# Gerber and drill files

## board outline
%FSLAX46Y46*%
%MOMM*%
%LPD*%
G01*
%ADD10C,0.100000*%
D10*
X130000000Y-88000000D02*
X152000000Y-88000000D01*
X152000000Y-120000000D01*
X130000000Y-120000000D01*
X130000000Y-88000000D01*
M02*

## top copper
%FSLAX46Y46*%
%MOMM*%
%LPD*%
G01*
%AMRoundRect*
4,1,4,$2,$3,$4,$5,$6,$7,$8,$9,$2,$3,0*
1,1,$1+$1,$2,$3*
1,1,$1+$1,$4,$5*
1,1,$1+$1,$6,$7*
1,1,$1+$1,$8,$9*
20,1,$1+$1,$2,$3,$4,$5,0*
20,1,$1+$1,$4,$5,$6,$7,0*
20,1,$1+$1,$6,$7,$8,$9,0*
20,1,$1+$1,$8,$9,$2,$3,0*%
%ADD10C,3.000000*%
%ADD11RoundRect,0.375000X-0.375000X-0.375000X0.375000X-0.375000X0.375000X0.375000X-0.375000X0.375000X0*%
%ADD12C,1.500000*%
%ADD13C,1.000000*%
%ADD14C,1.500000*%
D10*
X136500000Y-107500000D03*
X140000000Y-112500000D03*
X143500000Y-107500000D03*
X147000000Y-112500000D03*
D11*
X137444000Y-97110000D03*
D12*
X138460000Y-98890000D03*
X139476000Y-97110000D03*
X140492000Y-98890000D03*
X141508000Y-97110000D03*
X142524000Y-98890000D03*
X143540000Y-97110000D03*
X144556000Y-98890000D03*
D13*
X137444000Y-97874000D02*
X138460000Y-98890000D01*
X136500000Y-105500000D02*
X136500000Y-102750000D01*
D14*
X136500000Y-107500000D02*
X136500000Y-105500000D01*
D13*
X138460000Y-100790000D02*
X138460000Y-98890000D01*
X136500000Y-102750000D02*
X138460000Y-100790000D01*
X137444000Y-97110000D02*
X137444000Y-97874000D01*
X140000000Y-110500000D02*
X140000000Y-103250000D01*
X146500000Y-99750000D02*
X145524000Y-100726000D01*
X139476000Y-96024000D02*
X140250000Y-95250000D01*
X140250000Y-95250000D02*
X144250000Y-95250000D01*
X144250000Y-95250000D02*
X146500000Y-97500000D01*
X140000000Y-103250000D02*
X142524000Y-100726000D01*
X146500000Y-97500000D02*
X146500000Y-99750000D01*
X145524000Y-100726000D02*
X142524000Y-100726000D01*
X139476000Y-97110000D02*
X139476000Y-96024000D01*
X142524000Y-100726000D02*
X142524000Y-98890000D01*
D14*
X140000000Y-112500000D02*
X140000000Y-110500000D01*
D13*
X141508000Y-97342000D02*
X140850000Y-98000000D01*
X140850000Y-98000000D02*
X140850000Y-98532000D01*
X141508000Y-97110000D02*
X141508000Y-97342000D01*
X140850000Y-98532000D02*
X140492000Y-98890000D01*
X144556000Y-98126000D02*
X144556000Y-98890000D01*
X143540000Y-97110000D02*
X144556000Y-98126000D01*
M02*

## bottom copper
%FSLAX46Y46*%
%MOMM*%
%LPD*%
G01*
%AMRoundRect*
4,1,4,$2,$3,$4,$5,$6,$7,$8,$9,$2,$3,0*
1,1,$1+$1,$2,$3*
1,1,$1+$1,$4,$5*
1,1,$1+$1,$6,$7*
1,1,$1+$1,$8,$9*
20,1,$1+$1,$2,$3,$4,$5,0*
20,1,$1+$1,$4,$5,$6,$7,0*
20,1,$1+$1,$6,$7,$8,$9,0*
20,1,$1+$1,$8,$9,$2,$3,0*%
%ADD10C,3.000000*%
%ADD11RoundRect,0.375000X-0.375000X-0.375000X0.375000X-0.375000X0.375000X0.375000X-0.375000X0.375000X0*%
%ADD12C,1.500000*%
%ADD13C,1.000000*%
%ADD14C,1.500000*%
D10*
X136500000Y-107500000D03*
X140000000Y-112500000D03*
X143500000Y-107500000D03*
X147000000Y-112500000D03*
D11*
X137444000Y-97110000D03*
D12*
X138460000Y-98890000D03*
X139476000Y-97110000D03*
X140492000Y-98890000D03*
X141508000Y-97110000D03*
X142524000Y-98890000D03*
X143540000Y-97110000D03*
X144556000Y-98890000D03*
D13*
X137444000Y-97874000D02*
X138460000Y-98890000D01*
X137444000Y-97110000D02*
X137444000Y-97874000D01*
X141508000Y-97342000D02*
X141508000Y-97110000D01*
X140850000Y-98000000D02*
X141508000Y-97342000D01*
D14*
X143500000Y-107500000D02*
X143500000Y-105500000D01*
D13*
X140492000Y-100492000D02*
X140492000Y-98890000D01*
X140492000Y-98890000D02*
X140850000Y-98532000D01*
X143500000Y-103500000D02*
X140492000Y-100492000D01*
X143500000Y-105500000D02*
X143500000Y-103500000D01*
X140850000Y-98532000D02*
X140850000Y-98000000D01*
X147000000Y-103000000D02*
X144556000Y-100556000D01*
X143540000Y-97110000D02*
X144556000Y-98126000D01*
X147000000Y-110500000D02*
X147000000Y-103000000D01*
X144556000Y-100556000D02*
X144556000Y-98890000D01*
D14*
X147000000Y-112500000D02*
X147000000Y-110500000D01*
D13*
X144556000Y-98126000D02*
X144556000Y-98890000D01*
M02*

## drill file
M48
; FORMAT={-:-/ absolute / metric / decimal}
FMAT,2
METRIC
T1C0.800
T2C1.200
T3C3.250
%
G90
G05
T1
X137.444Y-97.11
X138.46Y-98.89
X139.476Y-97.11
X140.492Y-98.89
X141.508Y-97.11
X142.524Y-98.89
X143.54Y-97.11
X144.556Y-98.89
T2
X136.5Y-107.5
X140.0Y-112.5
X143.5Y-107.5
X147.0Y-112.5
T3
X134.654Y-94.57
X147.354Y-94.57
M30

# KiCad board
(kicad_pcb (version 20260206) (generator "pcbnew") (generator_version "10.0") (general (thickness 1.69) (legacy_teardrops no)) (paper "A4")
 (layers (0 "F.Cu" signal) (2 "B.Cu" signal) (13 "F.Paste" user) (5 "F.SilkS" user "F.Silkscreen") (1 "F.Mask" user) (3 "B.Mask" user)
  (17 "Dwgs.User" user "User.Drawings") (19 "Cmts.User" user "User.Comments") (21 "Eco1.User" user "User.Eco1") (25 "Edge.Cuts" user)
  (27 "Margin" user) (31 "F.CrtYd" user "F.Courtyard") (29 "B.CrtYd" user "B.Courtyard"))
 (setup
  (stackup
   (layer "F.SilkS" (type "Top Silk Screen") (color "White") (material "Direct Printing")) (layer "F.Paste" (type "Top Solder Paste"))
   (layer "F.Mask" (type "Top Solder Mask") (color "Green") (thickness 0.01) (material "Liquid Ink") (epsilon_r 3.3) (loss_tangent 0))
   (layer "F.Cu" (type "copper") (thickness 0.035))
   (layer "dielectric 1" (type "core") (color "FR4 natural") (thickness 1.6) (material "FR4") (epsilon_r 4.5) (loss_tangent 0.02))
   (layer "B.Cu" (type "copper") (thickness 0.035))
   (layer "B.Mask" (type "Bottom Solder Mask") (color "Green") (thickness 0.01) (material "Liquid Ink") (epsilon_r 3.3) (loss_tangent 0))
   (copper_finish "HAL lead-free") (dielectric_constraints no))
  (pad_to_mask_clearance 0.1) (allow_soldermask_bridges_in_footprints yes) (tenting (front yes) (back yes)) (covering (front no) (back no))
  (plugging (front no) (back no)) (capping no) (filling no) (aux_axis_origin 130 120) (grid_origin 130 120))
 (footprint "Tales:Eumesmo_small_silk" (layer "F.Cu") (at 148.5 101 90)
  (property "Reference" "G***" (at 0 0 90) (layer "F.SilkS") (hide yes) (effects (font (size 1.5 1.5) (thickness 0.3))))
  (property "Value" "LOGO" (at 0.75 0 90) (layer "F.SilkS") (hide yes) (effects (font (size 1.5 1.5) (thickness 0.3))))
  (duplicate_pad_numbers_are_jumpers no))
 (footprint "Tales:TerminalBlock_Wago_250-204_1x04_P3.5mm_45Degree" (layer "F.Cu") (at 141.75 110)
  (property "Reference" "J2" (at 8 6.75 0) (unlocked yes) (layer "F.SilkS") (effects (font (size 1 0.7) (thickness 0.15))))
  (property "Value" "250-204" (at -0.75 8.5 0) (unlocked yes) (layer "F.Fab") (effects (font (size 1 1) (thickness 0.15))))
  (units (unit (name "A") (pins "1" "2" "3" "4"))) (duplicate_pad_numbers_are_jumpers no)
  (pad "1" thru_hole circle (at -5.25 -2.5) (size 3 3) (drill 1.2) (layers "*.Cu" "*.Mask") (remove_unused_layers no) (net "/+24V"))
  (pad "2" thru_hole circle (at -1.75 2.5) (size 3 3) (drill 1.2) (layers "*.Cu" "*.Mask") (remove_unused_layers no) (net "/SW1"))
  (pad "3" thru_hole circle (at 1.75 -2.5) (size 3 3) (drill 1.2) (layers "*.Cu" "*.Mask") (remove_unused_layers no) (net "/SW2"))
  (pad "4" thru_hole circle (at 5.25 2.5) (size 3 3) (drill 1.2) (layers "*.Cu" "*.Mask") (remove_unused_layers no) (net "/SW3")))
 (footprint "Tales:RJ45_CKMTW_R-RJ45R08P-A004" (layer "F.Cu") (at 141 98 180)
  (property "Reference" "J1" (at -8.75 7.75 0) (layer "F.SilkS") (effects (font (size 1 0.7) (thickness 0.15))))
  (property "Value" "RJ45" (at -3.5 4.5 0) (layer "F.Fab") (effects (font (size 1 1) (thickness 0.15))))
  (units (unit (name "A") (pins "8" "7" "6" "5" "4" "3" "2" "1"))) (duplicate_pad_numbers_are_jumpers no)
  (pad "" np_thru_hole circle (at -6.354 3.43) (size 3.25 3.25) (drill 3.25) (layers "*.Cu" "*.Mask"))
  (pad "" np_thru_hole circle (at 6.346 3.43) (size 3.25 3.25) (drill 3.25) (layers "*.Cu" "*.Mask"))
  (pad "1" thru_hole roundrect (at 3.556 0.89) (size 1.5 1.5) (drill 0.8) (layers "*.Cu" "*.Mask") (remove_unused_layers no)
   (roundrect_rratio 0.25) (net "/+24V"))
  (pad "2" thru_hole circle (at 2.54 -0.89) (size 1.5 1.5) (drill 0.8) (layers "*.Cu" "*.Mask") (remove_unused_layers no) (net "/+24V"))
  (pad "3" thru_hole circle (at 1.524 0.89) (size 1.5 1.5) (drill 0.8) (layers "*.Cu" "*.Mask") (remove_unused_layers no) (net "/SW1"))
  (pad "4" thru_hole circle (at 0.508 -0.89) (size 1.5 1.5) (drill 0.8) (layers "*.Cu" "*.Mask") (remove_unused_layers no) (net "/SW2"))
  (pad "5" thru_hole circle (at -0.508 0.89) (size 1.5 1.5) (drill 0.8) (layers "*.Cu" "*.Mask") (remove_unused_layers no) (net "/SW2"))
  (pad "6" thru_hole circle (at -1.524 -0.89) (size 1.5 1.5) (drill 0.8) (layers "*.Cu" "*.Mask") (remove_unused_layers no) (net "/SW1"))
  (pad "7" thru_hole circle (at -2.54 0.89) (size 1.5 1.5) (drill 0.8) (layers "*.Cu" "*.Mask") (remove_unused_layers no) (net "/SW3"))
  (pad "8" thru_hole circle (at -3.556 -0.89) (size 1.5 1.5) (drill 0.8) (layers "*.Cu" "*.Mask") (remove_unused_layers no) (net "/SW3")))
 (gr_rect (start 130 88) (end 152 120) (stroke (width 0.1) (type default)) (fill no) (layer "Edge.Cuts"))
 (segment (start 137.444 97.874) (end 138.46 98.89) (width 1) (layer "F.Cu") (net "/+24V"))
 (segment (start 136.5 105.5) (end 136.5 102.75) (width 1) (layer "F.Cu") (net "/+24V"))
 (segment (start 136.5 107.5) (end 136.5 105.5) (width 1.5) (layer "F.Cu") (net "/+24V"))
 (segment (start 138.46 100.79) (end 138.46 98.89) (width 1) (layer "F.Cu") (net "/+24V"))
 (segment (start 136.5 102.75) (end 138.46 100.79) (width 1) (layer "F.Cu") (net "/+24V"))
 (segment (start 137.444 97.11) (end 137.444 97.874) (width 1) (layer "F.Cu") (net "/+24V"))
 (segment (start 137.444 97.874) (end 138.46 98.89) (width 1) (layer "B.Cu") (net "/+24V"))
 (segment (start 137.444 97.11) (end 137.444 97.874) (width 1) (layer "B.Cu") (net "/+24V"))
 (segment (start 140 110.5) (end 140 103.25) (width 1) (layer "F.Cu") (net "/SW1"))
 (segment (start 146.5 99.75) (end 145.524 100.726) (width 1) (layer "F.Cu") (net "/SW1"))
 (segment (start 139.476 96.024) (end 140.25 95.25) (width 1) (layer "F.Cu") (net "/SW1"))
 (segment (start 140.25 95.25) (end 144.25 95.25) (width 1) (layer "F.Cu") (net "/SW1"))
 (segment (start 144.25 95.25) (end 146.5 97.5) (width 1) (layer "F.Cu") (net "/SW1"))
 (segment (start 140 103.25) (end 142.524 100.726) (width 1) (layer "F.Cu") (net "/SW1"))
 (segment (start 146.5 97.5) (end 146.5 99.75) (width 1) (layer "F.Cu") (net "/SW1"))
 (segment (start 145.524 100.726) (end 142.524 100.726) (width 1) (layer "F.Cu") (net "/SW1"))
 (segment (start 139.476 97.11) (end 139.476 96.024) (width 1) (layer "F.Cu") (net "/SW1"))
 (segment (start 142.524 100.726) (end 142.524 98.89) (width 1) (layer "F.Cu") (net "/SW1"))
 (segment (start 140 112.5) (end 140 110.5) (width 1.5) (layer "F.Cu") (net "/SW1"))
 (segment (start 141.508 97.342) (end 140.85 98) (width 1) (layer "F.Cu") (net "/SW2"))
 (segment (start 140.85 98) (end 140.85 98.532) (width 1) (layer "F.Cu") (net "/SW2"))
 (segment (start 141.508 97.11) (end 141.508 97.342) (width 1) (layer "F.Cu") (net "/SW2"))
 (segment (start 140.85 98.532) (end 140.492 98.89) (width 1) (layer "F.Cu") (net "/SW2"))
 (segment (start 141.508 97.342) (end 141.508 97.11) (width 1) (layer "B.Cu") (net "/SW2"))
 (segment (start 140.85 98) (end 141.508 97.342) (width 1) (layer "B.Cu") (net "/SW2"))
 (segment (start 143.5 107.5) (end 143.5 105.5) (width 1.5) (layer "B.Cu") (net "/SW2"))
 (segment (start 140.492 100.492) (end 140.492 98.89) (width 1) (layer "B.Cu") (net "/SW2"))
 (segment (start 140.492 98.89) (end 140.85 98.532) (width 1) (layer "B.Cu") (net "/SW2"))
 (segment (start 143.5 103.5) (end 140.492 100.492) (width 1) (layer "B.Cu") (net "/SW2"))
 (segment (start 143.5 105.5) (end 143.5 103.5) (width 1) (layer "B.Cu") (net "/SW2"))
 (segment (start 140.85 98.532) (end 140.85 98) (width 1) (layer "B.Cu") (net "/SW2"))
 (segment (start 144.556 98.126) (end 144.556 98.89) (width 1) (layer "F.Cu") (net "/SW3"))
 (segment (start 143.54 97.11) (end 144.556 98.126) (width 1) (layer "F.Cu") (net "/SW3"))
 (segment (start 147 103) (end 144.556 100.556) (width 1) (layer "B.Cu") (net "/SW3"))
 (segment (start 143.54 97.11) (end 144.556 98.126) (width 1) (layer "B.Cu") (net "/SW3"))
 (segment (start 147 110.5) (end 147 103) (width 1) (layer "B.Cu") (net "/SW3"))
 (segment (start 144.556 100.556) (end 144.556 98.89) (width 1) (layer "B.Cu") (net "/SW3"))
 (segment (start 147 112.5) (end 147 110.5) (width 1.5) (layer "B.Cu") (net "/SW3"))
 (segment (start 144.556 98.126) (end 144.556 98.89) (width 1) (layer "B.Cu") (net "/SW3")))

